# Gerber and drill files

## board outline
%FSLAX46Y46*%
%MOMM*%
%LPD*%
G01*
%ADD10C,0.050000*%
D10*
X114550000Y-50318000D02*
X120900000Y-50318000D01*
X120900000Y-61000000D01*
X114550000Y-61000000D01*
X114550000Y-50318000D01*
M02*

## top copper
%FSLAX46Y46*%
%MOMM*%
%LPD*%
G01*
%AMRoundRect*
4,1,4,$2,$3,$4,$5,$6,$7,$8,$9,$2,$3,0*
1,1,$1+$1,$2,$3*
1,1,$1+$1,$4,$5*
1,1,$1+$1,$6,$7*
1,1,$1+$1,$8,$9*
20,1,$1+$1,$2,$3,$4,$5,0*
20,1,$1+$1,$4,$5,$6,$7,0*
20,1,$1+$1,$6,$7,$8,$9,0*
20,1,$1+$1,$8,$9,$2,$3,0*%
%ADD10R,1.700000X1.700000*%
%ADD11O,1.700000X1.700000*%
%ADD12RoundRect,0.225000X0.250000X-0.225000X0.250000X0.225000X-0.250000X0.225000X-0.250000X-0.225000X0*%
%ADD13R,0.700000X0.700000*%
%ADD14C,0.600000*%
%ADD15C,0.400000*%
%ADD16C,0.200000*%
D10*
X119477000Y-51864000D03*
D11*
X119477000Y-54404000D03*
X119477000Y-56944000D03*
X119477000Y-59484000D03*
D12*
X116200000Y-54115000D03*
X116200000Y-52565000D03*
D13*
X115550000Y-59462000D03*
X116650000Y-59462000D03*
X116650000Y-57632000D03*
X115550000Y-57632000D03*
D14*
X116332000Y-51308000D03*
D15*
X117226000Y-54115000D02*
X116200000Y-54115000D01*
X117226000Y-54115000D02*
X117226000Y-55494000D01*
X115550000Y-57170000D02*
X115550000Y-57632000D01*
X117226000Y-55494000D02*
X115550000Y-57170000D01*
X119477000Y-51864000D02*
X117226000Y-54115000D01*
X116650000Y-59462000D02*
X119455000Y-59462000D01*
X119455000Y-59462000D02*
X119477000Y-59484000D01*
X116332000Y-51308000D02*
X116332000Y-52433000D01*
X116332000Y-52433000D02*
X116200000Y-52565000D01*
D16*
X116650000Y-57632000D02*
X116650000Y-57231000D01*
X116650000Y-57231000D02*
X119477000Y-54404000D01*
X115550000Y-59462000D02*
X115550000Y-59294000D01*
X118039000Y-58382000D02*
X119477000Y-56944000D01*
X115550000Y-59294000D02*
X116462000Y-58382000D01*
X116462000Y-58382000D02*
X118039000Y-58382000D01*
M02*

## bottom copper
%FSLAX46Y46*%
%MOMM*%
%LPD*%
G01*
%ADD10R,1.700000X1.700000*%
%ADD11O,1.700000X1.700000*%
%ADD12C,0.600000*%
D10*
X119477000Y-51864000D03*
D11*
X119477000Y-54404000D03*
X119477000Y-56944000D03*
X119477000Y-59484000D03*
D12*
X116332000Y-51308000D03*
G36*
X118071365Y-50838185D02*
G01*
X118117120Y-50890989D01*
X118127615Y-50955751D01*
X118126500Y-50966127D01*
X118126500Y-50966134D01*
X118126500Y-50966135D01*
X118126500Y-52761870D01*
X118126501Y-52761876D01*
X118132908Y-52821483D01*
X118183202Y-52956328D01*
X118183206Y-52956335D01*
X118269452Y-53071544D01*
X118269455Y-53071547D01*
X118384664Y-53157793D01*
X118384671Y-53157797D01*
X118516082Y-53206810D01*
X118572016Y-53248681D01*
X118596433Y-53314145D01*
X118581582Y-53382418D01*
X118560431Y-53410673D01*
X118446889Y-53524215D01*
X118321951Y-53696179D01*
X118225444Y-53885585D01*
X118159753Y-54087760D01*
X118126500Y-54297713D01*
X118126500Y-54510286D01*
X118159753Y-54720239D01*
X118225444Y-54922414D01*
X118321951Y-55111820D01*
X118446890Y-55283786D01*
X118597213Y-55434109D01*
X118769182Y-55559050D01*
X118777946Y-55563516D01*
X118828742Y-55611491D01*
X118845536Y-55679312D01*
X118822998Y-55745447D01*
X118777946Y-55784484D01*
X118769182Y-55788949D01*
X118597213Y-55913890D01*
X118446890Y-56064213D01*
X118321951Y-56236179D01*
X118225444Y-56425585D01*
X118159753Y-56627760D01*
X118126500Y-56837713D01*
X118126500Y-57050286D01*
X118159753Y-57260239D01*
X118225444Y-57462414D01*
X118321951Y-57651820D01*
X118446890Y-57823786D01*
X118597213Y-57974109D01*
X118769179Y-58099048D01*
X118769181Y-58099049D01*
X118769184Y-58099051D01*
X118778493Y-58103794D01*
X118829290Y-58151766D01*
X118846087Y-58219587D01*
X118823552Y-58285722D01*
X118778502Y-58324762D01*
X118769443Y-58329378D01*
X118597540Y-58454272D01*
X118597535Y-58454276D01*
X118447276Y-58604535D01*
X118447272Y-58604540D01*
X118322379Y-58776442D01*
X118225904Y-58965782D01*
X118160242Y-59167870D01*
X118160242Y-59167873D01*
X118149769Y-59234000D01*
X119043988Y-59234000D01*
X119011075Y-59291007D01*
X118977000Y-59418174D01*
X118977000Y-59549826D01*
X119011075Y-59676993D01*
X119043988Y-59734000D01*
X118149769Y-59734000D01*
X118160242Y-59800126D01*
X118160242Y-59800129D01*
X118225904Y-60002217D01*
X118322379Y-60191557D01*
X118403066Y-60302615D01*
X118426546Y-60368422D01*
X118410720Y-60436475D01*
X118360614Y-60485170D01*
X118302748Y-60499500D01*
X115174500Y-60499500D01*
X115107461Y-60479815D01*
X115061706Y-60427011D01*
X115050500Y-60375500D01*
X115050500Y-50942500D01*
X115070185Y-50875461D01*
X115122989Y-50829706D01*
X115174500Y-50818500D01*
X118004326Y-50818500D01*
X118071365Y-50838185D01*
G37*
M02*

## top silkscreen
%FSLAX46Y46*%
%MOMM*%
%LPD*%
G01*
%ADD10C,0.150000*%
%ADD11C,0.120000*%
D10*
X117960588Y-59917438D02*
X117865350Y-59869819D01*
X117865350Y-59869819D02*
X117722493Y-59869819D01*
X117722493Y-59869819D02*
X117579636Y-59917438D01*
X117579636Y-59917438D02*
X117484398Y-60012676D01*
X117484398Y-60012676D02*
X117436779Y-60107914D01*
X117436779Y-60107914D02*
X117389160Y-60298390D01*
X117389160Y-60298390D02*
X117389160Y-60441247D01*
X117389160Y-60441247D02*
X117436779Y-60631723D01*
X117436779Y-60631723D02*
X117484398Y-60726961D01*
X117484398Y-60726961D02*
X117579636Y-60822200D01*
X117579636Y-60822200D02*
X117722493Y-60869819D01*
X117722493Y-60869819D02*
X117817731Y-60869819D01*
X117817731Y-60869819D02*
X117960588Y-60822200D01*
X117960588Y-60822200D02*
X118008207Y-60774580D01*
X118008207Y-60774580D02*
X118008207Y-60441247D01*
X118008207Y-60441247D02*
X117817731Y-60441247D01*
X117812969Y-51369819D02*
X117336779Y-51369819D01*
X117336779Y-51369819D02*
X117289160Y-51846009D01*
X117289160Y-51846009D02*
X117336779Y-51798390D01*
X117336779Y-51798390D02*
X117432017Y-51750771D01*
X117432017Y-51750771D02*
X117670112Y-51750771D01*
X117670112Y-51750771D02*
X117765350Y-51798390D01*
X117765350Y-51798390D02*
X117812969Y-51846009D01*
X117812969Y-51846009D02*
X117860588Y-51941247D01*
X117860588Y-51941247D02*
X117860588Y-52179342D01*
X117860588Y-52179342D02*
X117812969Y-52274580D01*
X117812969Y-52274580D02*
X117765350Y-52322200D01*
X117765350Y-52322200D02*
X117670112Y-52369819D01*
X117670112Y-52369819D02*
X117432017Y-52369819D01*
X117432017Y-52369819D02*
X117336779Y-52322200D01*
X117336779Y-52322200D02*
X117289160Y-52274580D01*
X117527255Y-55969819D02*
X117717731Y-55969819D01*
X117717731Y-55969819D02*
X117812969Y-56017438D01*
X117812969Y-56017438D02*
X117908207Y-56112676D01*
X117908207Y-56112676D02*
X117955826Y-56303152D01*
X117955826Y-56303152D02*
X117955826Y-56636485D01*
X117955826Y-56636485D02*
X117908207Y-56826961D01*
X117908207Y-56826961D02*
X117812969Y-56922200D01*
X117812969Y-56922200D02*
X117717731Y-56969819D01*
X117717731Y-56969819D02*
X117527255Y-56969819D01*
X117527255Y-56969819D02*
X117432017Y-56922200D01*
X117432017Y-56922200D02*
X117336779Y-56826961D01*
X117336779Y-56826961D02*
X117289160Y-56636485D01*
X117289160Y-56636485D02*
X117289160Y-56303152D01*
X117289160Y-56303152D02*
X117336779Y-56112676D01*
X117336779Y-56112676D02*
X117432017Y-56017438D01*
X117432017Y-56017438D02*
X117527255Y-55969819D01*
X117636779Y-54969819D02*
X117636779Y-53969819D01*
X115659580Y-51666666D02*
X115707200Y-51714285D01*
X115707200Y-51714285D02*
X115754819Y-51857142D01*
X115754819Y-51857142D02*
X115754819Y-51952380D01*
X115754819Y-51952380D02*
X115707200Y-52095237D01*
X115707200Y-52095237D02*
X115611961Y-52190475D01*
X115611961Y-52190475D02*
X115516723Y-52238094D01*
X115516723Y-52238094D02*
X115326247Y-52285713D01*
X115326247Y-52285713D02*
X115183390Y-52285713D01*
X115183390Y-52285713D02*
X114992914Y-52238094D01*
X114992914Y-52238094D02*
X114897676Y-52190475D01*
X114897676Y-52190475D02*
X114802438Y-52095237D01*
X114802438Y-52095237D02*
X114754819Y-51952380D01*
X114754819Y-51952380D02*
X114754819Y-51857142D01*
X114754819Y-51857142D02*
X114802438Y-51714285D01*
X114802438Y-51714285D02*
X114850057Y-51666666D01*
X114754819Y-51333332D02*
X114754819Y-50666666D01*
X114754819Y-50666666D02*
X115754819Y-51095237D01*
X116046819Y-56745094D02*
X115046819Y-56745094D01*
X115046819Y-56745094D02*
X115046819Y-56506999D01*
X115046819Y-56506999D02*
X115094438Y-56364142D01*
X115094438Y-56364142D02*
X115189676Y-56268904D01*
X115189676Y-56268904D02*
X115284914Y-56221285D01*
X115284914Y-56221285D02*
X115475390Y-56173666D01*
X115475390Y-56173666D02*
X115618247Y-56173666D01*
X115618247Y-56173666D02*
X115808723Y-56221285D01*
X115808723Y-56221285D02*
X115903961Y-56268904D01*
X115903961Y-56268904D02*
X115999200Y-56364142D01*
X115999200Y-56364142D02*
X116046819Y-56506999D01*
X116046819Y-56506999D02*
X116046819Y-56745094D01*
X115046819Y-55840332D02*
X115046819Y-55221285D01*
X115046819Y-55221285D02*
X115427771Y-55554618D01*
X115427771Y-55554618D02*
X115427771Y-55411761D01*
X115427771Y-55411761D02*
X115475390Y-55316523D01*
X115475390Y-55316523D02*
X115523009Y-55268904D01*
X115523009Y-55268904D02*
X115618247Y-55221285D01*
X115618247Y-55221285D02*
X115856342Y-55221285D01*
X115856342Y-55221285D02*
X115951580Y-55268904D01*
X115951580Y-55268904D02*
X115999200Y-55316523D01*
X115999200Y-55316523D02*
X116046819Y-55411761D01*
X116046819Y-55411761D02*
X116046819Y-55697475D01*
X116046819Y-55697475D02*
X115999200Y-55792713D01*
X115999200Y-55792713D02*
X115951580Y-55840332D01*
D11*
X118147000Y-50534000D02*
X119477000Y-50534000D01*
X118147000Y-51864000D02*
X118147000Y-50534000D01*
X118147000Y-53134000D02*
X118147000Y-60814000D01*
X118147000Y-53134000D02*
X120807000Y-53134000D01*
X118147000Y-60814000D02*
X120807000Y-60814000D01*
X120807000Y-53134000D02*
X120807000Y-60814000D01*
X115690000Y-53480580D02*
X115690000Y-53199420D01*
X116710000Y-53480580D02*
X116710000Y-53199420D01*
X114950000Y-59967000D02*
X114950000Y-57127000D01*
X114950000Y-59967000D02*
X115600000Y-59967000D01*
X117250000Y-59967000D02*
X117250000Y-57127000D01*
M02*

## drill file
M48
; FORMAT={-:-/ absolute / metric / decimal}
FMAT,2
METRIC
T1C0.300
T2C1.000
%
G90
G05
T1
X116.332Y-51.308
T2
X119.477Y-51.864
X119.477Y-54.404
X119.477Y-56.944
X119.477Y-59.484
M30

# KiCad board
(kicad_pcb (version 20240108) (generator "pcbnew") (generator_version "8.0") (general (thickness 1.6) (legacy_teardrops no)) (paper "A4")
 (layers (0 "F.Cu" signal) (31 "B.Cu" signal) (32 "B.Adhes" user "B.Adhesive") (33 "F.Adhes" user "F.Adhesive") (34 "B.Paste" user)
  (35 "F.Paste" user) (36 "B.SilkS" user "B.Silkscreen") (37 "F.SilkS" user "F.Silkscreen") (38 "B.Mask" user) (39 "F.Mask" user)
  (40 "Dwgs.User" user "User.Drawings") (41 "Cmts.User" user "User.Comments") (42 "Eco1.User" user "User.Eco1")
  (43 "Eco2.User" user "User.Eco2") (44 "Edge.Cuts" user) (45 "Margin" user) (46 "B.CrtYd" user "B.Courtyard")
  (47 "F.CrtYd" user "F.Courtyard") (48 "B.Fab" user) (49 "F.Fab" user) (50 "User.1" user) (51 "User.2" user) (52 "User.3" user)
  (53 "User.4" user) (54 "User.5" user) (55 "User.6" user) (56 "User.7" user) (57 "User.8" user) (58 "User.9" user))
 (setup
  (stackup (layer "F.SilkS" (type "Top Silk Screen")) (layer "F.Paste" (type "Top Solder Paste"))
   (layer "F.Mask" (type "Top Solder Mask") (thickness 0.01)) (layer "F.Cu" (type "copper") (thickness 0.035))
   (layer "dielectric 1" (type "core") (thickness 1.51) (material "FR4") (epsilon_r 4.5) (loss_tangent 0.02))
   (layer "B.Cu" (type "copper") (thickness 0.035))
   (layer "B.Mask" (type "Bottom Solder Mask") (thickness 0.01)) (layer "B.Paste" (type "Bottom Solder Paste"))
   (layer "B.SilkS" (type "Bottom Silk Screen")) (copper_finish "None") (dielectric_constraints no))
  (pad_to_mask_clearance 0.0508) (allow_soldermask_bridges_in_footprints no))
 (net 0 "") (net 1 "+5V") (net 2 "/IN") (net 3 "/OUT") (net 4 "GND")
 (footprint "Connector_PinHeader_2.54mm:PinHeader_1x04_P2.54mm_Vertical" (layer "F.Cu") (at 119.477 51.864)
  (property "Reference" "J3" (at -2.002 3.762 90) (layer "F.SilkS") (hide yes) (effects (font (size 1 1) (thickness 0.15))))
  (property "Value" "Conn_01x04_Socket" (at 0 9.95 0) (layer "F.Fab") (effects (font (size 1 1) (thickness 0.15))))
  (fp_line (start -1.33 -1.33) (end 0 -1.33) (stroke (width 0.12) (type solid)) (layer "F.SilkS"))
  (fp_line (start -1.33 0) (end -1.33 -1.33) (stroke (width 0.12) (type solid)) (layer "F.SilkS"))
  (fp_line (start -1.33 1.27) (end -1.33 8.95) (stroke (width 0.12) (type solid)) (layer "F.SilkS"))
  (fp_line (start -1.33 1.27) (end 1.33 1.27) (stroke (width 0.12) (type solid)) (layer "F.SilkS"))
  (fp_line (start -1.33 8.95) (end 1.33 8.95) (stroke (width 0.12) (type solid)) (layer "F.SilkS"))
  (fp_line (start 1.33 1.27) (end 1.33 8.95) (stroke (width 0.12) (type solid)) (layer "F.SilkS"))
  (pad "1" thru_hole rect (at 0 0) (size 1.7 1.7) (drill 1) (layers "*.Cu" "*.Mask") (remove_unused_layers no) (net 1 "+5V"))
  (pad "2" thru_hole oval (at 0 2.54) (size 1.7 1.7) (drill 1) (layers "*.Cu" "*.Mask") (remove_unused_layers no) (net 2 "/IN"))
  (pad "3" thru_hole oval (at 0 5.08) (size 1.7 1.7) (drill 1) (layers "*.Cu" "*.Mask") (remove_unused_layers no) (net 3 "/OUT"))
  (pad "4" thru_hole oval (at 0 7.62) (size 1.7 1.7) (drill 1) (layers "*.Cu" "*.Mask") (remove_unused_layers no) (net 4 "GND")))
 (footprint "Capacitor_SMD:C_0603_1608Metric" (layer "F.Cu") (at 116.2 53.34 90)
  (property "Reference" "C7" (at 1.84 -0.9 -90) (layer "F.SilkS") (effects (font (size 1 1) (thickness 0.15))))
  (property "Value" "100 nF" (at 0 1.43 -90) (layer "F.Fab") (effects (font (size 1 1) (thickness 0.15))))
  (fp_line (start -0.14058 -0.51) (end 0.14058 -0.51) (stroke (width 0.12) (type solid)) (layer "F.SilkS"))
  (fp_line (start -0.14058 0.51) (end 0.14058 0.51) (stroke (width 0.12) (type solid)) (layer "F.SilkS"))
  (pad "1" smd roundrect (at -0.775 0 90) (size 0.9 0.95) (layers "F.Cu" "F.Paste" "F.Mask") (roundrect_rratio 0.25) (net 1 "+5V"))
  (pad "2" smd roundrect (at 0.775 0 90) (size 0.9 0.95) (layers "F.Cu" "F.Paste" "F.Mask") (roundrect_rratio 0.25) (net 4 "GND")))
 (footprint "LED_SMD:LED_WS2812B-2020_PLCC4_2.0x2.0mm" (layer "F.Cu") (at 116.1 58.547 90)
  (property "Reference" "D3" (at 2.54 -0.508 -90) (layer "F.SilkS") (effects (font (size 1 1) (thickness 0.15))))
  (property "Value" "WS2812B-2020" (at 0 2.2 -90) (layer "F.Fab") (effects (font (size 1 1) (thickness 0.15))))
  (fp_line (start -1.42 -1.15) (end 1.42 -1.15) (stroke (width 0.12) (type solid)) (layer "F.SilkS"))
  (fp_line (start -1.42 -1.15) (end -1.42 -0.5) (stroke (width 0.12) (type solid)) (layer "F.SilkS"))
  (fp_line (start -1.42 1.15) (end 1.42 1.15) (stroke (width 0.12) (type solid)) (layer "F.SilkS"))
  (pad "1" smd rect (at -0.915 -0.55 90) (size 0.7 0.7) (layers "F.Cu" "F.Paste" "F.Mask") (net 3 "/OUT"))
  (pad "2" smd rect (at -0.915 0.55 90) (size 0.7 0.7) (layers "F.Cu" "F.Paste" "F.Mask") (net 4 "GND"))
  (pad "3" smd rect (at 0.915 0.55 90) (size 0.7 0.7) (layers "F.Cu" "F.Paste" "F.Mask") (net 2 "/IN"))
  (pad "4" smd rect (at 0.915 -0.55 90) (size 0.7 0.7) (layers "F.Cu" "F.Paste" "F.Mask") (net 1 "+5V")))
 (gr_rect (start 114.55 50.318) (end 120.9 61) (stroke (width 0.05) (type default)) (fill none) (layer "Edge.Cuts"))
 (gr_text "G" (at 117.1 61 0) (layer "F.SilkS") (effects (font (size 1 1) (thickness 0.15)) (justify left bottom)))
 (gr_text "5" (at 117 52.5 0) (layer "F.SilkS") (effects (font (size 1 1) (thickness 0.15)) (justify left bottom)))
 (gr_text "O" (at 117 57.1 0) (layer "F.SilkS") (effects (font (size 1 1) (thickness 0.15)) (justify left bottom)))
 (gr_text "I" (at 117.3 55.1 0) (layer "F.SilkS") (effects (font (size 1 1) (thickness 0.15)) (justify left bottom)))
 (segment (start 117.226 54.115) (end 116.2 54.115) (width 0.4) (layer "F.Cu") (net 1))
 (segment (start 117.226 54.115) (end 117.226 55.494) (width 0.4) (layer "F.Cu") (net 1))
 (segment (start 115.55 57.17) (end 115.55 57.632) (width 0.4) (layer "F.Cu") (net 1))
 (segment (start 117.226 55.494) (end 115.55 57.17) (width 0.4) (layer "F.Cu") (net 1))
 (segment (start 119.477 51.864) (end 117.226 54.115) (width 0.4) (layer "F.Cu") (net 1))
 (segment (start 116.65 59.462) (end 119.455 59.462) (width 0.4) (layer "F.Cu") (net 4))
 (segment (start 119.455 59.462) (end 119.477 59.484) (width 0.4) (layer "F.Cu") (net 4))
 (segment (start 116.332 51.308) (end 116.332 52.433) (width 0.4) (layer "F.Cu") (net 4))
 (segment (start 116.332 52.433) (end 116.2 52.565) (width 0.4) (layer "F.Cu") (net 4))
 (via (at 116.332 51.308) (size 0.6) (drill 0.3) (layers "F.Cu" "B.Cu") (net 4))
 (segment (start 116.65 57.632) (end 116.65 57.231) (width 0.2) (layer "F.Cu") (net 2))
 (segment (start 116.65 57.231) (end 119.477 54.404) (width 0.2) (layer "F.Cu") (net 2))
 (segment (start 115.55 59.462) (end 115.55 59.294) (width 0.2) (layer "F.Cu") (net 3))
 (segment (start 118.039 58.382) (end 119.477 56.944) (width 0.2) (layer "F.Cu") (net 3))
 (segment (start 115.55 59.294) (end 116.462 58.382) (width 0.2) (layer "F.Cu") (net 3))
 (segment (start 116.462 58.382) (end 118.039 58.382) (width 0.2) (layer "F.Cu") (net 3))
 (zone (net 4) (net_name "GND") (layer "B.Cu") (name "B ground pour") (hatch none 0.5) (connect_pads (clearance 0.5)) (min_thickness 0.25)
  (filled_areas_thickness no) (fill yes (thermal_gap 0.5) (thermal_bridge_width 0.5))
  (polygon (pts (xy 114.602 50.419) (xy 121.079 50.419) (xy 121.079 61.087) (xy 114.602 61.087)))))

